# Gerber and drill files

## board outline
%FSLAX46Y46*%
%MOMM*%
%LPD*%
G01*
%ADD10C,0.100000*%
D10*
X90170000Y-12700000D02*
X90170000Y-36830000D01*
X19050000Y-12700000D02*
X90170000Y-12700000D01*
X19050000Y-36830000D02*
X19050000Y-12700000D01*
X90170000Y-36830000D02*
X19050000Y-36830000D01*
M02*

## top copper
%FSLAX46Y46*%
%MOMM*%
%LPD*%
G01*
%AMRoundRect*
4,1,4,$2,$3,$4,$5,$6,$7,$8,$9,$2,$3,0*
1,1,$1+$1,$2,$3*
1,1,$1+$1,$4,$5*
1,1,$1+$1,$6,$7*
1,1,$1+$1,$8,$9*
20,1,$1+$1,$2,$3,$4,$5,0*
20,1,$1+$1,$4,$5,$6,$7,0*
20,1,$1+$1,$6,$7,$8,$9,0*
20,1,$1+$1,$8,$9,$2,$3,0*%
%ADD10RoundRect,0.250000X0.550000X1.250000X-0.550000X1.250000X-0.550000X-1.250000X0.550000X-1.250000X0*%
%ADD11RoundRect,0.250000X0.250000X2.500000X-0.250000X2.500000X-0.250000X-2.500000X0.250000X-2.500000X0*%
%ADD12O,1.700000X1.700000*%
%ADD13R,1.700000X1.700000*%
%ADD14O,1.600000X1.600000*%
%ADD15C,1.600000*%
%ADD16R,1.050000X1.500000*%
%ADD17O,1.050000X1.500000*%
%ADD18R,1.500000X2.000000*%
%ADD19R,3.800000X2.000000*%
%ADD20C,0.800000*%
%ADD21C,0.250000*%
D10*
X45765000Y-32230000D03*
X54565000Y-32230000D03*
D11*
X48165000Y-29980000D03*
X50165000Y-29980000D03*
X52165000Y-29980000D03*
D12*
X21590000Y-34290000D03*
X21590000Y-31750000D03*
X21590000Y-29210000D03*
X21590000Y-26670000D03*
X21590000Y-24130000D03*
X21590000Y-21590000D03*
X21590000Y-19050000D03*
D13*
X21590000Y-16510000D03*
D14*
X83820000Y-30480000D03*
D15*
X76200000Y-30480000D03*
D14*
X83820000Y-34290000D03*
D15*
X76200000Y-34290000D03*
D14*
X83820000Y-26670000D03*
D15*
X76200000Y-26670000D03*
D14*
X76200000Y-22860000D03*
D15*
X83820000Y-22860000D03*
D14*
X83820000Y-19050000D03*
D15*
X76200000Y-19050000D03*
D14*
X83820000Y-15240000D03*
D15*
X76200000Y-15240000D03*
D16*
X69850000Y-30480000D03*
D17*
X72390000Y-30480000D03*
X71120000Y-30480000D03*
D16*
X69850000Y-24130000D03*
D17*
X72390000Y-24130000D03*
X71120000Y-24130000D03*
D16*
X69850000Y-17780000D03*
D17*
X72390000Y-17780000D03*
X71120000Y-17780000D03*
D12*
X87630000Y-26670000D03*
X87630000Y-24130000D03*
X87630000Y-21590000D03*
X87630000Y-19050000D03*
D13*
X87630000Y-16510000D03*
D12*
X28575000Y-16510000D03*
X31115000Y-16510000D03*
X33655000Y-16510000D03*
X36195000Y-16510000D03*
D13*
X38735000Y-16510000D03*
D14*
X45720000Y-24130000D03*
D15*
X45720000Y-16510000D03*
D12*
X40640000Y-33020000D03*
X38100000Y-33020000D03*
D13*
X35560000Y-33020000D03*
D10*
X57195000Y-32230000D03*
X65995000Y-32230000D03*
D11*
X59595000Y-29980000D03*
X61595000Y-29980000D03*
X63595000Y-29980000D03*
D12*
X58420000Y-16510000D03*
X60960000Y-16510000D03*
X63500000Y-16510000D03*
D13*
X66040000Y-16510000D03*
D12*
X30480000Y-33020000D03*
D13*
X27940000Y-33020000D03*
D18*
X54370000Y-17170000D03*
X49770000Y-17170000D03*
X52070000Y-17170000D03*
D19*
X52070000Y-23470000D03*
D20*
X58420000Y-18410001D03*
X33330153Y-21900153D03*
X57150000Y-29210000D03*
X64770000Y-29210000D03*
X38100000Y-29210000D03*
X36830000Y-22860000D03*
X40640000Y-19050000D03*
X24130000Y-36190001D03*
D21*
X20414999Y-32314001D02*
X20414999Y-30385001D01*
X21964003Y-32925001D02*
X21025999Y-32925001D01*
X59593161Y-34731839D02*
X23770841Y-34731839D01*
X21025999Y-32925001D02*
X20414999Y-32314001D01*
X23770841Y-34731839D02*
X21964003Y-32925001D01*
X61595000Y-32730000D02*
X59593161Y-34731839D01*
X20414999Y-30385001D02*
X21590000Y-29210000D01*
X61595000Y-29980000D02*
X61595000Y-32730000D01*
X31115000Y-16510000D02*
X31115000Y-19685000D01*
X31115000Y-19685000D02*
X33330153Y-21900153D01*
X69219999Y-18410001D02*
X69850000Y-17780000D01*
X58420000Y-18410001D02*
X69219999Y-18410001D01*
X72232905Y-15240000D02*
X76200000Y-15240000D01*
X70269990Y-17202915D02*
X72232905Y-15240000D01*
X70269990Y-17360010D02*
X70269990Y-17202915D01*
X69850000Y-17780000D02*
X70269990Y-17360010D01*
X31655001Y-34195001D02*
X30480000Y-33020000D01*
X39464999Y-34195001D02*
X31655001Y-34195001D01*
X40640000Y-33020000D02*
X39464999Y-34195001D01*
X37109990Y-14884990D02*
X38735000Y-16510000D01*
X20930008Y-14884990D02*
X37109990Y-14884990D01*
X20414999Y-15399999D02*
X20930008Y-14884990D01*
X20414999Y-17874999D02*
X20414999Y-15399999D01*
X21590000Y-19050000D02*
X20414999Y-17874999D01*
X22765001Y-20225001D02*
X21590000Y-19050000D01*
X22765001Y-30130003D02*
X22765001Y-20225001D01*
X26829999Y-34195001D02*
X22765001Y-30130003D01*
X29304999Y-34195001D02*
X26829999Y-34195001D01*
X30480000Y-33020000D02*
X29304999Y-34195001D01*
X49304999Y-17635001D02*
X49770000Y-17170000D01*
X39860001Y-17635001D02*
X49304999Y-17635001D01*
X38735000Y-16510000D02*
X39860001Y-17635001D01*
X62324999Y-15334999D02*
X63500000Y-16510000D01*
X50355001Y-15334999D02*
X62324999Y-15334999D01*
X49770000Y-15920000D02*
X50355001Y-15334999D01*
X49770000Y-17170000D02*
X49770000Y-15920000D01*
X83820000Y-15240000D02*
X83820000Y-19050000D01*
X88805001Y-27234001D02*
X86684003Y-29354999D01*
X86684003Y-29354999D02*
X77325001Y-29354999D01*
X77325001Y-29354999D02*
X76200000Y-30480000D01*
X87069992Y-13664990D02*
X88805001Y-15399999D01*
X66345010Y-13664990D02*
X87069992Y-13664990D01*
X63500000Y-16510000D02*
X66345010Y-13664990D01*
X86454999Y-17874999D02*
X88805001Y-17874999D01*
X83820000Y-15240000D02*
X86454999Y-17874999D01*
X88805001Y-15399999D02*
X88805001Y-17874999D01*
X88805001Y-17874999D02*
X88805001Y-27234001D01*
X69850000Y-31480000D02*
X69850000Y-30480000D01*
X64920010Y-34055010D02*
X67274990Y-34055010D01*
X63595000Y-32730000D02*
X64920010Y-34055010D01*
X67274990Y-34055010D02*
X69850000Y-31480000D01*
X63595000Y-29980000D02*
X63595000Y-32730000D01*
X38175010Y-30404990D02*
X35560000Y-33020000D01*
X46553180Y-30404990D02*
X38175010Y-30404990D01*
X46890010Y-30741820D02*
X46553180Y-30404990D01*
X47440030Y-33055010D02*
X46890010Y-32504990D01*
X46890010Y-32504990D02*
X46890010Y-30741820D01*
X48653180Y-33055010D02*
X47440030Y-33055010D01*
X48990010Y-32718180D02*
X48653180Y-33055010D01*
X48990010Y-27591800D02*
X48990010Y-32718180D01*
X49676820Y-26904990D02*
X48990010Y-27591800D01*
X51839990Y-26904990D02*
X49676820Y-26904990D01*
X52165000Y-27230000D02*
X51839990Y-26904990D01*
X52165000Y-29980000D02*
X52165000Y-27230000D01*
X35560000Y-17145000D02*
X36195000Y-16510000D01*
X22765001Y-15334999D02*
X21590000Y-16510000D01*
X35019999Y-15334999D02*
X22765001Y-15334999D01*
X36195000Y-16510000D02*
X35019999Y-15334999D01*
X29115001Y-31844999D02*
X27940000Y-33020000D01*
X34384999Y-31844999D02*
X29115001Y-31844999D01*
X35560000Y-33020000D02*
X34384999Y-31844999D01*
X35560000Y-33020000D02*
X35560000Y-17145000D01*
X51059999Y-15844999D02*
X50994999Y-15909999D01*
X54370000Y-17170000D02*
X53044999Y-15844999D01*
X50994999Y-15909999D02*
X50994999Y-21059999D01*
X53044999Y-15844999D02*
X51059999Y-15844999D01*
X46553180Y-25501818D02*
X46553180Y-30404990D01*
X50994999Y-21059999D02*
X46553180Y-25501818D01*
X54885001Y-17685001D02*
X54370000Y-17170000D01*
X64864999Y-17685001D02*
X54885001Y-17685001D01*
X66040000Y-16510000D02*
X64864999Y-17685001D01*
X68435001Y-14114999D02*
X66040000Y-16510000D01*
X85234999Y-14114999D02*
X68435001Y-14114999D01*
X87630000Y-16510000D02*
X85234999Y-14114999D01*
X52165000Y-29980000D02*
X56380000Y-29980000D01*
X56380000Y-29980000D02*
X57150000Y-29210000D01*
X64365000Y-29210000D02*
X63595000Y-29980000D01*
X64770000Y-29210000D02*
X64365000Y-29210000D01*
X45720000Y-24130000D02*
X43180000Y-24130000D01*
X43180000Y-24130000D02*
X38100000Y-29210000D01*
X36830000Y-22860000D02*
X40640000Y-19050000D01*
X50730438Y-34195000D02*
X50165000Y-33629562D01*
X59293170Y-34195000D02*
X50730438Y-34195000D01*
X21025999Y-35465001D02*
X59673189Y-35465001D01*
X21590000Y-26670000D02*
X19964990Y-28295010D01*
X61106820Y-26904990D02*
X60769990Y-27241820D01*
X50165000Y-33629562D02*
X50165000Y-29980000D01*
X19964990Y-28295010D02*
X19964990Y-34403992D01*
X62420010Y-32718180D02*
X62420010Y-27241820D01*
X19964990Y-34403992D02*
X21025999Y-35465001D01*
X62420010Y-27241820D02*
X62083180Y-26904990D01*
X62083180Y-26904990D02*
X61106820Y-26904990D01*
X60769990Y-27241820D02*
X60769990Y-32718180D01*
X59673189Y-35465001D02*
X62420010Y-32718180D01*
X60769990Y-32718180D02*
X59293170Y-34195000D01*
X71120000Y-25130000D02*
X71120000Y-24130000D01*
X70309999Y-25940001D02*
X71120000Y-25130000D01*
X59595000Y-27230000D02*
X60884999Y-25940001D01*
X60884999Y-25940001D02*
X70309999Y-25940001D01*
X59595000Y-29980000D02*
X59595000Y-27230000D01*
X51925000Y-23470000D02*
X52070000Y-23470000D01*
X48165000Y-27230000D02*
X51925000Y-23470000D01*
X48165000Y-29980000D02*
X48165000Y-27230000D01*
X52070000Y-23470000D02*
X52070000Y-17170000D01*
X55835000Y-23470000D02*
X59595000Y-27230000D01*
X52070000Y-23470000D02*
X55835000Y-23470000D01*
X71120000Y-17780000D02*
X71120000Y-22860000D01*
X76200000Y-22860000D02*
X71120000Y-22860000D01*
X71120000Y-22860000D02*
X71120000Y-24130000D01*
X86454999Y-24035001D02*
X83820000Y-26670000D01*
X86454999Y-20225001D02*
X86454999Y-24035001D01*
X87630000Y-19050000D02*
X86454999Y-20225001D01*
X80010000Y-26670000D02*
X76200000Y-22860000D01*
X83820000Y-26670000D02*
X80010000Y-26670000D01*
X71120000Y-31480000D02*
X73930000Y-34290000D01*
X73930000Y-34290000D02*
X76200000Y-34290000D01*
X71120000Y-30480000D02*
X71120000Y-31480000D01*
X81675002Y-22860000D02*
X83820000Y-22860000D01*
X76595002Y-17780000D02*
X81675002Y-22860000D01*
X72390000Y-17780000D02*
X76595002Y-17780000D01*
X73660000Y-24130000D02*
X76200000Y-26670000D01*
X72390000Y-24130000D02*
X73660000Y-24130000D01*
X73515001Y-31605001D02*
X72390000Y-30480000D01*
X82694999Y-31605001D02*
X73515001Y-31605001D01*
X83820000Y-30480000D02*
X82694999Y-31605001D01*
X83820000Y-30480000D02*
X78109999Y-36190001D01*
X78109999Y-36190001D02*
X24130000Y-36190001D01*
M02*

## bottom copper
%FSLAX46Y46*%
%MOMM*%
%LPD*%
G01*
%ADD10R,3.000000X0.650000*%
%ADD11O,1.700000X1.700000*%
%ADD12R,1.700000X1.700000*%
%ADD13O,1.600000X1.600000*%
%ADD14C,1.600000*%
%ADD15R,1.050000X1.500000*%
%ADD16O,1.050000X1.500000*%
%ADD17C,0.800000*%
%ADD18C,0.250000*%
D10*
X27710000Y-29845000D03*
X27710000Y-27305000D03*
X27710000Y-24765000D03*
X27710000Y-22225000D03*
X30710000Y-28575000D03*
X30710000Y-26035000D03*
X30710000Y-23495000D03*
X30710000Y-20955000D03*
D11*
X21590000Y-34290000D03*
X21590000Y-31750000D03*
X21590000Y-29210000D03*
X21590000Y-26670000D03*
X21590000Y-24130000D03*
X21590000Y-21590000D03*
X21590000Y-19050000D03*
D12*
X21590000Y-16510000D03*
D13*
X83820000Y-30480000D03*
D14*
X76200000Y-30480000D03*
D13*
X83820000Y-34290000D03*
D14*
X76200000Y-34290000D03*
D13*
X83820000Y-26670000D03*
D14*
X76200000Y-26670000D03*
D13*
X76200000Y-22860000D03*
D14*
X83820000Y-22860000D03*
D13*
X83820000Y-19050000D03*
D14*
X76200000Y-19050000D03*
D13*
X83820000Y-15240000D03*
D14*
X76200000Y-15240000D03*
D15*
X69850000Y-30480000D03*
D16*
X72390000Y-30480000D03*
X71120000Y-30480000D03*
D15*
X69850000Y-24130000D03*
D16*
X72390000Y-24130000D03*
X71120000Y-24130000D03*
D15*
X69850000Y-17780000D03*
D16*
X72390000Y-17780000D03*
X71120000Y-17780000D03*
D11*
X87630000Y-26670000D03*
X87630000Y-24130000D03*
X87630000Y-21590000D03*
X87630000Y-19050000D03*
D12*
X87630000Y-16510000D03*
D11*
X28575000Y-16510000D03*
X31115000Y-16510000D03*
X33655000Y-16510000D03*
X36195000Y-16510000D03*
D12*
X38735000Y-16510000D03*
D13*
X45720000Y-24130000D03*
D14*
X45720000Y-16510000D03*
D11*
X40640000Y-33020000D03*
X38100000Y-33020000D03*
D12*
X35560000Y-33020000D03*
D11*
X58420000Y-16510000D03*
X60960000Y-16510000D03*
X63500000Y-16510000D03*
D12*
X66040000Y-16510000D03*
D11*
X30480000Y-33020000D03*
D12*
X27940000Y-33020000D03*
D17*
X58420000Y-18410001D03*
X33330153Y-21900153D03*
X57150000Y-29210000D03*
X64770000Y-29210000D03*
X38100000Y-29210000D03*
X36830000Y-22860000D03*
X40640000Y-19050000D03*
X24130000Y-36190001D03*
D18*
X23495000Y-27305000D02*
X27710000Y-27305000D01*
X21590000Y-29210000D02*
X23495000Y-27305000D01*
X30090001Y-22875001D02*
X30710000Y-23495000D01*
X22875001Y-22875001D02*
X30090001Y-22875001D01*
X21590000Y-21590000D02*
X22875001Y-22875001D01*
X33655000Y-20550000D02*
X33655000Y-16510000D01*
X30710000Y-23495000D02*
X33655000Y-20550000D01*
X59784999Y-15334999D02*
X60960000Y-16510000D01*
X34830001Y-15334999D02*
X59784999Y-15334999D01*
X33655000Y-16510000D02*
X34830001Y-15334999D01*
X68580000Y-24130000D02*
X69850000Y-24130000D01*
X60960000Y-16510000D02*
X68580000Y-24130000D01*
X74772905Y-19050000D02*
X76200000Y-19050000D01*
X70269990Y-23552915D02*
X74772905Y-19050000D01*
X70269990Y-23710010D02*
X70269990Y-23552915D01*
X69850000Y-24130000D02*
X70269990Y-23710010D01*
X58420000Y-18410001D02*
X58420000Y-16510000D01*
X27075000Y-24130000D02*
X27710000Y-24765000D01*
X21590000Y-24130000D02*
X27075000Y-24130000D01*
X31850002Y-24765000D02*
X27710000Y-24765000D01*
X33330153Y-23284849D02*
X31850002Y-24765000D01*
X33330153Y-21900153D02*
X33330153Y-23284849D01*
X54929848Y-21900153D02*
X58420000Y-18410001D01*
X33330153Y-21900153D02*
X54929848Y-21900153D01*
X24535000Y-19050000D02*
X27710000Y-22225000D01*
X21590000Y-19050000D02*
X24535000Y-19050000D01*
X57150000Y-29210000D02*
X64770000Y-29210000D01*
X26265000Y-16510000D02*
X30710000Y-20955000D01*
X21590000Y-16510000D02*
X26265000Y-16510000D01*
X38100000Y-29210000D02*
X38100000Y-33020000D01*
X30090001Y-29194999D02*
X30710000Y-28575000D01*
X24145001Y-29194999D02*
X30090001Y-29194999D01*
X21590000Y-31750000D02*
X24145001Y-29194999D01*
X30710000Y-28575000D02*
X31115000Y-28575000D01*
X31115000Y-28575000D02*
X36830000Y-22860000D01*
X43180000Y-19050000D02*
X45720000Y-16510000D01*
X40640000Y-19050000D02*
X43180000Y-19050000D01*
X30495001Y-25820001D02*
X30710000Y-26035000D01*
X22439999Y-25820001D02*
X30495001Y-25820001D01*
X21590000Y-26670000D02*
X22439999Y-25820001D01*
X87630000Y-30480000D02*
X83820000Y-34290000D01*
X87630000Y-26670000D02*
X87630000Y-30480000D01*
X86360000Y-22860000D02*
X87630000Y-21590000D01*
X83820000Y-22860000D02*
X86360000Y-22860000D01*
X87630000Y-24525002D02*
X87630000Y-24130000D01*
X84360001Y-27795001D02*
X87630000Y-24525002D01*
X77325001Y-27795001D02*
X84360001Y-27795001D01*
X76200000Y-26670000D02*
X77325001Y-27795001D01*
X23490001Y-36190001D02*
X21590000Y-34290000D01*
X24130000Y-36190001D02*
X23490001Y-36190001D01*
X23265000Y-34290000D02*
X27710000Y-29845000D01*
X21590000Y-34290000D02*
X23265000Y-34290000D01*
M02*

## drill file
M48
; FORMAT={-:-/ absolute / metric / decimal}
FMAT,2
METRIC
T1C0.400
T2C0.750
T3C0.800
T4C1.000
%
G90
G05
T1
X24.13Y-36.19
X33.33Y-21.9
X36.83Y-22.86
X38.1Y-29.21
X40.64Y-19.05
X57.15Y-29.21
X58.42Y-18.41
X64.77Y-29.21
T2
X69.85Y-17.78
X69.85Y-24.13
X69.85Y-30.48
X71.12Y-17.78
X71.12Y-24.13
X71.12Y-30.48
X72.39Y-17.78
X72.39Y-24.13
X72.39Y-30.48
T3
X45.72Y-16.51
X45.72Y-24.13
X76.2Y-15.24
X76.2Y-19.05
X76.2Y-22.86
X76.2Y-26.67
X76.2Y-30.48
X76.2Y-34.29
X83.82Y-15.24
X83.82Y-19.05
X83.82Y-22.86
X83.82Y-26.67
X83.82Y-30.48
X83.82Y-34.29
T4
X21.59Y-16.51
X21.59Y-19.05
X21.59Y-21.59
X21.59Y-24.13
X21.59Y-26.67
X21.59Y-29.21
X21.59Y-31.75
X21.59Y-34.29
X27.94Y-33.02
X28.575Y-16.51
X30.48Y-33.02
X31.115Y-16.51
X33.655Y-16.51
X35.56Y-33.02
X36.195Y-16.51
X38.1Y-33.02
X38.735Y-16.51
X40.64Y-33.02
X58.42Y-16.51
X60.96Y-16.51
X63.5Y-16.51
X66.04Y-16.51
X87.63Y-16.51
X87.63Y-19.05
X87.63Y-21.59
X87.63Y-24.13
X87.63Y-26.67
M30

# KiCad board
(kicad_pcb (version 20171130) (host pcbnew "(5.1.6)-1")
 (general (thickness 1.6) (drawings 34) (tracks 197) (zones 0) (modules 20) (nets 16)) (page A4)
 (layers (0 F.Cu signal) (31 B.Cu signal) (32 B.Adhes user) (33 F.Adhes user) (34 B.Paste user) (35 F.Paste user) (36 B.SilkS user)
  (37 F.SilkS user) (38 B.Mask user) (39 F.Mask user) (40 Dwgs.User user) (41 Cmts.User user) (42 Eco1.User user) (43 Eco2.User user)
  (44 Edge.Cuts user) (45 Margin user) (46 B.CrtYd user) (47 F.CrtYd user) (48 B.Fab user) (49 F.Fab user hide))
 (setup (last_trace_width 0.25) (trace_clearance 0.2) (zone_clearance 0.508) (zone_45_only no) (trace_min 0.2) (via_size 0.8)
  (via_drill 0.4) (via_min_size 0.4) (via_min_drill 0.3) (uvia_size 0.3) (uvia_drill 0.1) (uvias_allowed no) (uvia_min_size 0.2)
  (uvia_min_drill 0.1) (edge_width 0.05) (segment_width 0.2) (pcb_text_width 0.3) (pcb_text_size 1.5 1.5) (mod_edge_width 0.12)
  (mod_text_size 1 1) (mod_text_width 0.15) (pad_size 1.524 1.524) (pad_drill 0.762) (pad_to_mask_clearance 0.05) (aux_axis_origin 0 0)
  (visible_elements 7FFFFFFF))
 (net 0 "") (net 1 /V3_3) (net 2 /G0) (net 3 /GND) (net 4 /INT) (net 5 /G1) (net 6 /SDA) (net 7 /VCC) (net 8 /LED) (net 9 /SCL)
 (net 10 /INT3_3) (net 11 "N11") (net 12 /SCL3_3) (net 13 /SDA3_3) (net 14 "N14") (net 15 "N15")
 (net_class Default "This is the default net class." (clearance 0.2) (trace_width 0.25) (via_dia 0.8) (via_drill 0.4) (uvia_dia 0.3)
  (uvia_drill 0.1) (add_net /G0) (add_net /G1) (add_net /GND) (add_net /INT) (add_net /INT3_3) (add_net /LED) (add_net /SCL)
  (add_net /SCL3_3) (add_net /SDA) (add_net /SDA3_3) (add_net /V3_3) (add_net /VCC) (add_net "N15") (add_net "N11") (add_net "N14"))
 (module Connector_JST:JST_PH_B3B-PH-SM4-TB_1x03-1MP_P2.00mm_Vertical (layer F.Cu) (at 50.165 30.48 180)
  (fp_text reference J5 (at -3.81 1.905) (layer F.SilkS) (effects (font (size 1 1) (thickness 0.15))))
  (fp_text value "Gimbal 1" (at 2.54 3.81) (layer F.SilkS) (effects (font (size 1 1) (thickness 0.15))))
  (pad MP smd roundrect (at 4.4 -1.75 180) (size 1.6 3) (layers F.Cu F.Paste F.Mask) (roundrect_rratio 0.15625))
  (pad MP smd roundrect (at -4.4 -1.75 180) (size 1.6 3) (layers F.Cu F.Paste F.Mask) (roundrect_rratio 0.15625))
  (pad 3 smd roundrect (at 2 0.5 180) (size 1 5.5) (layers F.Cu F.Paste F.Mask) (roundrect_rratio 0.25) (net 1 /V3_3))
  (pad 2 smd roundrect (at 0 0.5 180) (size 1 5.5) (layers F.Cu F.Paste F.Mask) (roundrect_rratio 0.25) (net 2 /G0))
  (pad 1 smd roundrect (at -2 0.5 180) (size 1 5.5) (layers F.Cu F.Paste F.Mask) (roundrect_rratio 0.25) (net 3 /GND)))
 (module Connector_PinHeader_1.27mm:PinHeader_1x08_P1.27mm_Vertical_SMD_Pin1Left (layer B.Cu) (at 29.21 25.4 180)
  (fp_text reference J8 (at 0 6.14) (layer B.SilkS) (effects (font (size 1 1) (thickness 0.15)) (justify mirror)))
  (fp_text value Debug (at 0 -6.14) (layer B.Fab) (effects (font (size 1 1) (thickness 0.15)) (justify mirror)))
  (pad 8 smd rect (at 1.5 -4.445 180) (size 3 0.65) (layers B.Cu B.Paste B.Mask) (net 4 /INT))
  (pad 6 smd rect (at 1.5 -1.905 180) (size 3 0.65) (layers B.Cu B.Paste B.Mask) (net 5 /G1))
  (pad 4 smd rect (at 1.5 0.635 180) (size 3 0.65) (layers B.Cu B.Paste B.Mask) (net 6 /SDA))
  (pad 2 smd rect (at 1.5 3.175 180) (size 3 0.65) (layers B.Cu B.Paste B.Mask) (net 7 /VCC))
  (pad 7 smd rect (at -1.5 -3.175 180) (size 3 0.65) (layers B.Cu B.Paste B.Mask) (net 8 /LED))
  (pad 5 smd rect (at -1.5 -0.635 180) (size 3 0.65) (layers B.Cu B.Paste B.Mask) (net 2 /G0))
  (pad 3 smd rect (at -1.5 1.905 180) (size 3 0.65) (layers B.Cu B.Paste B.Mask) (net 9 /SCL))
  (pad 1 smd rect (at -1.5 4.445 180) (size 3 0.65) (layers B.Cu B.Paste B.Mask) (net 3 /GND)))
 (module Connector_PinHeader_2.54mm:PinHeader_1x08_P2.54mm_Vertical (layer F.Cu) (at 21.59 16.51)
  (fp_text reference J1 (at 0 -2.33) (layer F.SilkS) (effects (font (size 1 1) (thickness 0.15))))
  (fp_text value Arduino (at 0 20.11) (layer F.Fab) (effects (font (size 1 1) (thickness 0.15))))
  (pad 8 thru_hole oval (at 0 17.78) (size 1.7 1.7) (drill 1) (layers *.Cu *.Mask) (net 4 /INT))
  (pad 7 thru_hole oval (at 0 15.24) (size 1.7 1.7) (drill 1) (layers *.Cu *.Mask) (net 8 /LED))
  (pad 6 thru_hole oval (at 0 12.7) (size 1.7 1.7) (drill 1) (layers *.Cu *.Mask) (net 5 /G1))
  (pad 5 thru_hole oval (at 0 10.16) (size 1.7 1.7) (drill 1) (layers *.Cu *.Mask) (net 2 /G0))
  (pad 4 thru_hole oval (at 0 7.62) (size 1.7 1.7) (drill 1) (layers *.Cu *.Mask) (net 6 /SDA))
  (pad 3 thru_hole oval (at 0 5.08) (size 1.7 1.7) (drill 1) (layers *.Cu *.Mask) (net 9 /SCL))
  (pad 2 thru_hole oval (at 0 2.54) (size 1.7 1.7) (drill 1) (layers *.Cu *.Mask) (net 7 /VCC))
  (pad 1 thru_hole rect (at 0 0) (size 1.7 1.7) (drill 1) (layers *.Cu *.Mask) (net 3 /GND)))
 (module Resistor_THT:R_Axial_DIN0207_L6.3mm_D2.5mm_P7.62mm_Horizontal (layer F.Cu) (at 76.2 30.48)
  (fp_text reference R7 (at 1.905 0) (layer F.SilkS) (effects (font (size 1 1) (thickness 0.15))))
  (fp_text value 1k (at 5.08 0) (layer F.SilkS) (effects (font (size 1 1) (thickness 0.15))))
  (pad 2 thru_hole oval (at 7.62 0) (size 1.6 1.6) (drill 0.8) (layers *.Cu *.Mask) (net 4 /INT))
  (pad 1 thru_hole circle (at 0 0) (size 1.6 1.6) (drill 0.8) (layers *.Cu *.Mask) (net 7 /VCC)))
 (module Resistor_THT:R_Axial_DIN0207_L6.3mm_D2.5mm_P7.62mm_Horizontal (layer F.Cu) (at 76.2 34.29)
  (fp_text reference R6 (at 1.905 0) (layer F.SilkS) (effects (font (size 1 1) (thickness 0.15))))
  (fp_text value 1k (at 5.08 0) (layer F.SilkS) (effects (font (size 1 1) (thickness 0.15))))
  (pad 2 thru_hole oval (at 7.62 0) (size 1.6 1.6) (drill 0.8) (layers *.Cu *.Mask) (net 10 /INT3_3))
  (pad 1 thru_hole circle (at 0 0) (size 1.6 1.6) (drill 0.8) (layers *.Cu *.Mask) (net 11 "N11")))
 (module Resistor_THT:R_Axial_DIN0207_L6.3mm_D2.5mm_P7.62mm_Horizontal (layer F.Cu) (at 76.2 26.67)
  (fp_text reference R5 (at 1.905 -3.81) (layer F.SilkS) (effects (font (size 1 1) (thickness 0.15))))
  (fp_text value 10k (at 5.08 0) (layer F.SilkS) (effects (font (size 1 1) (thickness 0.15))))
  (pad 2 thru_hole oval (at 7.62 0) (size 1.6 1.6) (drill 0.8) (layers *.Cu *.Mask) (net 1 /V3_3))
  (pad 1 thru_hole circle (at 0 0) (size 1.6 1.6) (drill 0.8) (layers *.Cu *.Mask) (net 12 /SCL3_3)))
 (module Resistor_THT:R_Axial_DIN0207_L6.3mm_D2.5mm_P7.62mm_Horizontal (layer F.Cu) (at 83.82 22.86 180)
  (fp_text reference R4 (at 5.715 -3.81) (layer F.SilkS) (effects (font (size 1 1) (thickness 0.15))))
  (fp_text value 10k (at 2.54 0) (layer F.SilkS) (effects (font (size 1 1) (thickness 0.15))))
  (pad 2 thru_hole oval (at 7.62 0 180) (size 1.6 1.6) (drill 0.8) (layers *.Cu *.Mask) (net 1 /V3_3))
  (pad 1 thru_hole circle (at 0 0 180) (size 1.6 1.6) (drill 0.8) (layers *.Cu *.Mask) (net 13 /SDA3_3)))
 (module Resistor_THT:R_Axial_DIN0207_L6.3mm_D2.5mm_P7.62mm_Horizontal (layer F.Cu) (at 76.2 19.05)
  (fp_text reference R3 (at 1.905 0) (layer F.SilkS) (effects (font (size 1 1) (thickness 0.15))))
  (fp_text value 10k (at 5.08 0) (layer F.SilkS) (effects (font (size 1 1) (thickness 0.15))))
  (pad 2 thru_hole oval (at 7.62 0) (size 1.6 1.6) (drill 0.8) (layers *.Cu *.Mask) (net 7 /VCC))
  (pad 1 thru_hole circle (at 0 0) (size 1.6 1.6) (drill 0.8) (layers *.Cu *.Mask) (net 9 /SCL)))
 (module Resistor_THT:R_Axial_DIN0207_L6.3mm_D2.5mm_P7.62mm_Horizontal (layer F.Cu) (at 76.2 15.24)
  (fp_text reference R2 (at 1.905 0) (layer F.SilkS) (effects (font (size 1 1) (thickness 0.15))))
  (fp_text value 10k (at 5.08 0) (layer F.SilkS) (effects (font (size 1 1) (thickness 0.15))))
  (pad 2 thru_hole oval (at 7.62 0) (size 1.6 1.6) (drill 0.8) (layers *.Cu *.Mask) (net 7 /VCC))
  (pad 1 thru_hole circle (at 0 0) (size 1.6 1.6) (drill 0.8) (layers *.Cu *.Mask) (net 6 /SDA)))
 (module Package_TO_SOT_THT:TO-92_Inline (layer F.Cu) (at 69.85 30.48)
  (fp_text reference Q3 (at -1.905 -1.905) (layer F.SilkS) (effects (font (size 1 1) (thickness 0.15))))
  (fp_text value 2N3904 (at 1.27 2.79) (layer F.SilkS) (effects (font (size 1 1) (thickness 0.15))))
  (pad 1 thru_hole rect (at 0 0) (size 1.05 1.5) (drill 0.75) (layers *.Cu *.Mask) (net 3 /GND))
  (pad 3 thru_hole oval (at 2.54 0) (size 1.05 1.5) (drill 0.75) (layers *.Cu *.Mask) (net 4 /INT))
  (pad 2 thru_hole oval (at 1.27 0) (size 1.05 1.5) (drill 0.75) (layers *.Cu *.Mask) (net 11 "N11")))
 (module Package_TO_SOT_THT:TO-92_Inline (layer F.Cu) (at 69.85 24.13)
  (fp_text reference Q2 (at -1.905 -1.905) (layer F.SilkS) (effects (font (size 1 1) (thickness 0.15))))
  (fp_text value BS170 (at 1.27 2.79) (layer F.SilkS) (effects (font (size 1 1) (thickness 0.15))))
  (pad 1 thru_hole rect (at 0 0) (size 1.05 1.5) (drill 0.75) (layers *.Cu *.Mask) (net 9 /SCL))
  (pad 3 thru_hole oval (at 2.54 0) (size 1.05 1.5) (drill 0.75) (layers *.Cu *.Mask) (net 12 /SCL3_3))
  (pad 2 thru_hole oval (at 1.27 0) (size 1.05 1.5) (drill 0.75) (layers *.Cu *.Mask) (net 1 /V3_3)))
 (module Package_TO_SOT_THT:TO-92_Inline (layer F.Cu) (at 69.85 17.78)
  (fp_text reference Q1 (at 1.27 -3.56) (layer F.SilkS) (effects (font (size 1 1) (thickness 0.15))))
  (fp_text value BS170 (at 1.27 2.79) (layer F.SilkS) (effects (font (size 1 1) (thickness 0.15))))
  (pad 1 thru_hole rect (at 0 0) (size 1.05 1.5) (drill 0.75) (layers *.Cu *.Mask) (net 6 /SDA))
  (pad 3 thru_hole oval (at 2.54 0) (size 1.05 1.5) (drill 0.75) (layers *.Cu *.Mask) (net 13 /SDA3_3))
  (pad 2 thru_hole oval (at 1.27 0) (size 1.05 1.5) (drill 0.75) (layers *.Cu *.Mask) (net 1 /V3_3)))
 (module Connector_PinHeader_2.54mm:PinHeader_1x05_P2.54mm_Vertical (layer F.Cu) (at 87.63 16.51)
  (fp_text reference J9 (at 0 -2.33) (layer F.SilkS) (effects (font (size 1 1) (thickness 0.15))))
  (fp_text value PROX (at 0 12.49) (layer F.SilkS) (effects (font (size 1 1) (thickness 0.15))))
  (pad 5 thru_hole oval (at 0 10.16) (size 1.7 1.7) (drill 1) (layers *.Cu *.Mask) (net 10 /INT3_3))
  (pad 4 thru_hole oval (at 0 7.62) (size 1.7 1.7) (drill 1) (layers *.Cu *.Mask) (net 12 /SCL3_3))
  (pad 3 thru_hole oval (at 0 5.08) (size 1.7 1.7) (drill 1) (layers *.Cu *.Mask) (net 13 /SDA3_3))
  (pad 2 thru_hole oval (at 0 2.54) (size 1.7 1.7) (drill 1) (layers *.Cu *.Mask) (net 1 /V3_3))
  (pad 1 thru_hole rect (at 0 0) (size 1.7 1.7) (drill 1) (layers *.Cu *.Mask) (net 3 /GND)))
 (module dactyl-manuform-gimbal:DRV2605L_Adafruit (layer F.Cu) (at 38.735 16.51 270)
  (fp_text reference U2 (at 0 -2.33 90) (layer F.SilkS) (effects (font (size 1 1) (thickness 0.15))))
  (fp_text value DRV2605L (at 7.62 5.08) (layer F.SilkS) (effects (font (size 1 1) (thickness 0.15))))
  (pad 5 thru_hole oval (at 0 10.16 270) (size 1.7 1.7) (drill 1) (layers *.Cu *.Mask) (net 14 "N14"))
  (pad 4 thru_hole oval (at 0 7.62 270) (size 1.7 1.7) (drill 1) (layers *.Cu *.Mask) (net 6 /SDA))
  (pad 3 thru_hole oval (at 0 5.08 270) (size 1.7 1.7) (drill 1) (layers *.Cu *.Mask) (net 9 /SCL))
  (pad 2 thru_hole oval (at 0 2.54 270) (size 1.7 1.7) (drill 1) (layers *.Cu *.Mask) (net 3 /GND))
  (pad 1 thru_hole rect (at 0 0 270) (size 1.7 1.7) (drill 1) (layers *.Cu *.Mask) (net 7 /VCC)))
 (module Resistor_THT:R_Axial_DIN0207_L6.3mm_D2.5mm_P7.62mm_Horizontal (layer F.Cu) (at 45.72 16.51 270)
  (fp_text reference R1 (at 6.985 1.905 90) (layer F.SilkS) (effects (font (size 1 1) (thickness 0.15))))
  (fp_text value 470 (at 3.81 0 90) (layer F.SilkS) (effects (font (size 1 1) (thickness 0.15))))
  (pad 2 thru_hole oval (at 7.62 0 270) (size 1.6 1.6) (drill 0.8) (layers *.Cu *.Mask) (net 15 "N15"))
  (pad 1 thru_hole circle (at 0 0 270) (size 1.6 1.6) (drill 0.8) (layers *.Cu *.Mask) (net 8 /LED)))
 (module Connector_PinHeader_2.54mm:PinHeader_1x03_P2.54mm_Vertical (layer F.Cu) (at 35.56 33.02 90)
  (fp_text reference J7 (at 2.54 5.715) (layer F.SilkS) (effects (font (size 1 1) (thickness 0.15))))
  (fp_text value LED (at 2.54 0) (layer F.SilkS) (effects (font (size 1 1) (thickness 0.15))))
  (pad 3 thru_hole oval (at 0 5.08 90) (size 1.7 1.7) (drill 1) (layers *.Cu *.Mask) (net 7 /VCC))
  (pad 2 thru_hole oval (at 0 2.54 90) (size 1.7 1.7) (drill 1) (layers *.Cu *.Mask) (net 15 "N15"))
  (pad 1 thru_hole rect (at 0 0 90) (size 1.7 1.7) (drill 1) (layers *.Cu *.Mask) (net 3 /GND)))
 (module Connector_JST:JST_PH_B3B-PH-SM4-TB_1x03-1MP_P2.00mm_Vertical (layer F.Cu) (at 61.595 30.48 180)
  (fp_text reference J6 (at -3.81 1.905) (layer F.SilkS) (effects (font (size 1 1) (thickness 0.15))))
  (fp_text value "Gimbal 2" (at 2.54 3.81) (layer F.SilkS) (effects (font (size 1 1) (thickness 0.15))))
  (pad MP smd roundrect (at 4.4 -1.75 180) (size 1.6 3) (layers F.Cu F.Paste F.Mask) (roundrect_rratio 0.15625))
  (pad MP smd roundrect (at -4.4 -1.75 180) (size 1.6 3) (layers F.Cu F.Paste F.Mask) (roundrect_rratio 0.15625))
  (pad 3 smd roundrect (at 2 0.5 180) (size 1 5.5) (layers F.Cu F.Paste F.Mask) (roundrect_rratio 0.25) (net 1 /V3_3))
  (pad 2 smd roundrect (at 0 0.5 180) (size 1 5.5) (layers F.Cu F.Paste F.Mask) (roundrect_rratio 0.25) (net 5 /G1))
  (pad 1 smd roundrect (at -2 0.5 180) (size 1 5.5) (layers F.Cu F.Paste F.Mask) (roundrect_rratio 0.25) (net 3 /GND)))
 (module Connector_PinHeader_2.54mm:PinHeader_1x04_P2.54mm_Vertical (layer F.Cu) (at 66.04 16.51 270)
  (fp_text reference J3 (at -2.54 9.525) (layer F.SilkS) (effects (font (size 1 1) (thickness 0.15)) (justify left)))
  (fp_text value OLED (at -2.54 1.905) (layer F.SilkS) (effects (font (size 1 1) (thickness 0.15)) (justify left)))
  (pad 4 thru_hole oval (at 0 7.62 270) (size 1.7 1.7) (drill 1) (layers *.Cu *.Mask) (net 6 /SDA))
  (pad 3 thru_hole oval (at 0 5.08 270) (size 1.7 1.7) (drill 1) (layers *.Cu *.Mask) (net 9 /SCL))
  (pad 2 thru_hole oval (at 0 2.54 270) (size 1.7 1.7) (drill 1) (layers *.Cu *.Mask) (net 7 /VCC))
  (pad 1 thru_hole rect (at 0 0 270) (size 1.7 1.7) (drill 1) (layers *.Cu *.Mask) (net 3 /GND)))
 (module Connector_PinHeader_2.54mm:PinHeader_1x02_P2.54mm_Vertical (layer F.Cu) (at 27.94 33.02 90)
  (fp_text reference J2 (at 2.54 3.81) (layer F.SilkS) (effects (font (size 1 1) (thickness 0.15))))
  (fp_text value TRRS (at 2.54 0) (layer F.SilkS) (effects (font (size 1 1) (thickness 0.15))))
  (pad 2 thru_hole oval (at 0 2.54 90) (size 1.7 1.7) (drill 1) (layers *.Cu *.Mask) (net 7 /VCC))
  (pad 1 thru_hole rect (at 0 0 90) (size 1.7 1.7) (drill 1) (layers *.Cu *.Mask) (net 3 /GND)))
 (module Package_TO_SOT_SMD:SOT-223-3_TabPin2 (layer F.Cu) (at 52.07 20.32 270)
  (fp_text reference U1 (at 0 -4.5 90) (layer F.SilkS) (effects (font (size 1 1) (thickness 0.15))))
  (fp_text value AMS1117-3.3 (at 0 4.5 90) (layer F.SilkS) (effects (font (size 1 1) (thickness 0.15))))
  (pad 1 smd rect (at -3.15 -2.3 270) (size 2 1.5) (layers F.Cu F.Paste F.Mask) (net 3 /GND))
  (pad 3 smd rect (at -3.15 2.3 270) (size 2 1.5) (layers F.Cu F.Paste F.Mask) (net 7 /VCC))
  (pad 2 smd rect (at -3.15 0 270) (size 2 1.5) (layers F.Cu F.Paste F.Mask) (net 1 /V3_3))
  (pad 2 smd rect (at 3.15 0 270) (size 2 3.8) (layers F.Cu F.Paste F.Mask) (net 1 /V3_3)))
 (gr_line (start 90.17 12.7) (end 90.17 36.83) (layer Edge.Cuts) (width 0.1))
 (gr_line (start 19.05 12.7) (end 90.17 12.7) (layer Edge.Cuts) (width 0.1))
 (gr_line (start 19.05 36.83) (end 19.05 12.7) (layer Edge.Cuts) (width 0.1))
 (gr_line (start 90.17 36.83) (end 19.05 36.83) (layer Edge.Cuts) (width 0.1))
 (segment (start 20.414999 32.314001) (end 20.414999 30.385001) (width 0.25) (layer F.Cu) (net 5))
 (segment (start 21.964003 32.925001) (end 21.025999 32.925001) (width 0.25) (layer F.Cu) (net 5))
 (segment (start 59.593161 34.731839) (end 23.770841 34.731839) (width 0.25) (layer F.Cu) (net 5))
 (segment (start 21.025999 32.925001) (end 20.414999 32.314001) (width 0.25) (layer F.Cu) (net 5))
 (segment (start 23.770841 34.731839) (end 21.964003 32.925001) (width 0.25) (layer F.Cu) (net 5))
 (segment (start 61.595 32.73) (end 59.593161 34.731839) (width 0.25) (layer F.Cu) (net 5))
 (segment (start 20.414999 30.385001) (end 21.59 29.21) (width 0.25) (layer F.Cu) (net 5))
 (segment (start 61.595 29.98) (end 61.595 32.73) (width 0.25) (layer F.Cu) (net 5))
 (segment (start 23.495 27.305) (end 27.71 27.305) (width 0.25) (layer B.Cu) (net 5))
 (segment (start 21.59 29.21) (end 23.495 27.305) (width 0.25) (layer B.Cu) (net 5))
 (segment (start 30.090001 22.875001) (end 30.71 23.495) (width 0.25) (layer B.Cu) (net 9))
 (segment (start 22.875001 22.875001) (end 30.090001 22.875001) (width 0.25) (layer B.Cu) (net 9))
 (segment (start 21.59 21.59) (end 22.875001 22.875001) (width 0.25) (layer B.Cu) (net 9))
 (segment (start 33.655 20.55) (end 33.655 16.51) (width 0.25) (layer B.Cu) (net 9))
 (segment (start 30.71 23.495) (end 33.655 20.55) (width 0.25) (layer B.Cu) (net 9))
 (segment (start 59.784999 15.334999) (end 60.96 16.51) (width 0.25) (layer B.Cu) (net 9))
 (segment (start 34.830001 15.334999) (end 59.784999 15.334999) (width 0.25) (layer B.Cu) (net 9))
 (segment (start 33.655 16.51) (end 34.830001 15.334999) (width 0.25) (layer B.Cu) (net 9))
 (segment (start 68.58 24.13) (end 69.85 24.13) (width 0.25) (layer B.Cu) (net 9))
 (segment (start 60.96 16.51) (end 68.58 24.13) (width 0.25) (layer B.Cu) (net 9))
 (segment (start 74.772905 19.05) (end 76.2 19.05) (width 0.25) (layer B.Cu) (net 9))
 (segment (start 70.26999 23.552915) (end 74.772905 19.05) (width 0.25) (layer B.Cu) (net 9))
 (segment (start 70.26999 23.71001) (end 70.26999 23.552915) (width 0.25) (layer B.Cu) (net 9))
 (segment (start 69.85 24.13) (end 70.26999 23.71001) (width 0.25) (layer B.Cu) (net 9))
 (via (at 58.42 18.410001) (size 0.8) (drill 0.4) (layers F.Cu B.Cu) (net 6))
 (segment (start 58.42 18.410001) (end 58.42 16.51) (width 0.25) (layer B.Cu) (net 6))
 (segment (start 27.075 24.13) (end 27.71 24.765) (width 0.25) (layer B.Cu) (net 6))
 (segment (start 21.59 24.13) (end 27.075 24.13) (width 0.25) (layer B.Cu) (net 6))
 (via (at 33.330153 21.900153) (size 0.8) (drill 0.4) (layers F.Cu B.Cu) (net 6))
 (segment (start 31.115 16.51) (end 31.115 19.685) (width 0.25) (layer F.Cu) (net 6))
 (segment (start 31.115 19.685) (end 33.330153 21.900153) (width 0.25) (layer F.Cu) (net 6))
 (segment (start 31.850002 24.765) (end 27.71 24.765) (width 0.25) (layer B.Cu) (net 6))
 (segment (start 33.330153 23.284849) (end 31.850002 24.765) (width 0.25) (layer B.Cu) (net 6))
 (segment (start 33.330153 21.900153) (end 33.330153 23.284849) (width 0.25) (layer B.Cu) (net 6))
 (segment (start 54.929848 21.900153) (end 58.42 18.410001) (width 0.25) (layer B.Cu) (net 6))
 (segment (start 33.330153 21.900153) (end 54.929848 21.900153) (width 0.25) (layer B.Cu) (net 6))
 (segment (start 69.219999 18.410001) (end 69.85 17.78) (width 0.25) (layer F.Cu) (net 6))
 (segment (start 58.42 18.410001) (end 69.219999 18.410001) (width 0.25) (layer F.Cu) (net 6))
 (segment (start 72.232905 15.24) (end 76.2 15.24) (width 0.25) (layer F.Cu) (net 6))
 (segment (start 70.26999 17.202915) (end 72.232905 15.24) (width 0.25) (layer F.Cu) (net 6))
 (segment (start 70.26999 17.36001) (end 70.26999 17.202915) (width 0.25) (layer F.Cu) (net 6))
 (segment (start 69.85 17.78) (end 70.26999 17.36001) (width 0.25) (layer F.Cu) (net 6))
 (segment (start 31.655001 34.195001) (end 30.48 33.02) (width 0.25) (layer F.Cu) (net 7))
 (segment (start 39.464999 34.195001) (end 31.655001 34.195001) (width 0.25) (layer F.Cu) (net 7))
 (segment (start 40.64 33.02) (end 39.464999 34.195001) (width 0.25) (layer F.Cu) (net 7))
 (segment (start 37.10999 14.88499) (end 38.735 16.51) (width 0.25) (layer F.Cu) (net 7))
 (segment (start 20.930008 14.88499) (end 37.10999 14.88499) (width 0.25) (layer F.Cu) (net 7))
 (segment (start 20.414999 15.399999) (end 20.930008 14.88499) (width 0.25) (layer F.Cu) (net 7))
 (segment (start 20.414999 17.874999) (end 20.414999 15.399999) (width 0.25) (layer F.Cu) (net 7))
 (segment (start 21.59 19.05) (end 20.414999 17.874999) (width 0.25) (layer F.Cu) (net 7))
 (segment (start 22.765001 20.225001) (end 21.59 19.05) (width 0.25) (layer F.Cu) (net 7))
 (segment (start 22.765001 30.130003) (end 22.765001 20.225001) (width 0.25) (layer F.Cu) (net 7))
 (segment (start 26.829999 34.195001) (end 22.765001 30.130003) (width 0.25) (layer F.Cu) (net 7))
 (segment (start 29.304999 34.195001) (end 26.829999 34.195001) (width 0.25) (layer F.Cu) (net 7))
 (segment (start 30.48 33.02) (end 29.304999 34.195001) (width 0.25) (layer F.Cu) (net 7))
 (segment (start 49.304999 17.635001) (end 49.77 17.17) (width 0.25) (layer F.Cu) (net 7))
 (segment (start 39.860001 17.635001) (end 49.304999 17.635001) (width 0.25) (layer F.Cu) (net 7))
 (segment (start 38.735 16.51) (end 39.860001 17.635001) (width 0.25) (layer F.Cu) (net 7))
 (segment (start 62.324999 15.334999) (end 63.5 16.51) (width 0.25) (layer F.Cu) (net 7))
 (segment (start 50.355001 15.334999) (end 62.324999 15.334999) (width 0.25) (layer F.Cu) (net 7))
 (segment (start 49.77 15.92) (end 50.355001 15.334999) (width 0.25) (layer F.Cu) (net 7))
 (segment (start 49.77 17.17) (end 49.77 15.92) (width 0.25) (layer F.Cu) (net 7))
 (segment (start 83.82 15.24) (end 83.82 19.05) (width 0.25) (layer F.Cu) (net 7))
 (segment (start 88.805001 27.234001) (end 86.684003 29.354999) (width 0.25) (layer F.Cu) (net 7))
 (segment (start 86.684003 29.354999) (end 77.325001 29.354999) (width 0.25) (layer F.Cu) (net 7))
 (segment (start 77.325001 29.354999) (end 76.2 30.48) (width 0.25) (layer F.Cu) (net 7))
 (segment (start 87.069992 13.66499) (end 88.805001 15.399999) (width 0.25) (layer F.Cu) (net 7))
 (segment (start 66.34501 13.66499) (end 87.069992 13.66499) (width 0.25) (layer F.Cu) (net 7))
 (segment (start 63.5 16.51) (end 66.34501 13.66499) (width 0.25) (layer F.Cu) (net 7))
 (segment (start 86.454999 17.874999) (end 88.805001 17.874999) (width 0.25) (layer F.Cu) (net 7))
 (segment (start 83.82 15.24) (end 86.454999 17.874999) (width 0.25) (layer F.Cu) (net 7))
 (segment (start 88.805001 15.399999) (end 88.805001 17.874999) (width 0.25) (layer F.Cu) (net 7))
 (segment (start 88.805001 17.874999) (end 88.805001 27.234001) (width 0.25) (layer F.Cu) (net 7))
 (segment (start 24.535 19.05) (end 27.71 22.225) (width 0.25) (layer B.Cu) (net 7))
 (segment (start 21.59 19.05) (end 24.535 19.05) (width 0.25) (layer B.Cu) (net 7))
 (segment (start 69.85 31.48) (end 69.85 30.48) (width 0.25) (layer F.Cu) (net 3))
 (segment (start 64.92001 34.05501) (end 67.27499 34.05501) (width 0.25) (layer F.Cu) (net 3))
 (segment (start 63.595 32.73) (end 64.92001 34.05501) (width 0.25) (layer F.Cu) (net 3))
 (segment (start 67.27499 34.05501) (end 69.85 31.48) (width 0.25) (layer F.Cu) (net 3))
 (segment (start 63.595 29.98) (end 63.595 32.73) (width 0.25) (layer F.Cu) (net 3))
 (segment (start 38.17501 30.40499) (end 35.56 33.02) (width 0.25) (layer F.Cu) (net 3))
 (segment (start 46.55318 30.40499) (end 38.17501 30.40499) (width 0.25) (layer F.Cu) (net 3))
 (segment (start 46.89001 30.74182) (end 46.55318 30.40499) (width 0.25) (layer F.Cu) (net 3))
 (segment (start 47.44003 33.05501) (end 46.89001 32.50499) (width 0.25) (layer F.Cu) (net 3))
 (segment (start 46.89001 32.50499) (end 46.89001 30.74182) (width 0.25) (layer F.Cu) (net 3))
 (segment (start 48.65318 33.05501) (end 47.44003 33.05501) (width 0.25) (layer F.Cu) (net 3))
 (segment (start 48.99001 32.71818) (end 48.65318 33.05501) (width 0.25) (layer F.Cu) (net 3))
 (segment (start 48.99001 27.5918) (end 48.99001 32.71818) (width 0.25) (layer F.Cu) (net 3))
 (segment (start 49.67682 26.90499) (end 48.99001 27.5918) (width 0.25) (layer F.Cu) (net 3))
 (segment (start 51.83999 26.90499) (end 49.67682 26.90499) (width 0.25) (layer F.Cu) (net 3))
 (segment (start 52.165 27.23) (end 51.83999 26.90499) (width 0.25) (layer F.Cu) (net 3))
 (segment (start 52.165 29.98) (end 52.165 27.23) (width 0.25) (layer F.Cu) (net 3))
 (segment (start 35.56 17.145) (end 36.195 16.51) (width 0.25) (layer F.Cu) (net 3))
 (segment (start 22.765001 15.334999) (end 21.59 16.51) (width 0.25) (layer F.Cu) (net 3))
 (segment (start 35.019999 15.334999) (end 22.765001 15.334999) (width 0.25) (layer F.Cu) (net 3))
 (segment (start 36.195 16.51) (end 35.019999 15.334999) (width 0.25) (layer F.Cu) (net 3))
 (segment (start 29.115001 31.844999) (end 27.94 33.02) (width 0.25) (layer F.Cu) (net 3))
 (segment (start 34.384999 31.844999) (end 29.115001 31.844999) (width 0.25) (layer F.Cu) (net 3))
 (segment (start 35.56 33.02) (end 34.384999 31.844999) (width 0.25) (layer F.Cu) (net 3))
 (segment (start 35.56 33.02) (end 35.56 17.145) (width 0.25) (layer F.Cu) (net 3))
 (segment (start 51.059999 15.844999) (end 50.994999 15.909999) (width 0.25) (layer F.Cu) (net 3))
 (segment (start 54.37 17.17) (end 53.044999 15.844999) (width 0.25) (layer F.Cu) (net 3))
 (segment (start 50.994999 15.909999) (end 50.994999 21.059999) (width 0.25) (layer F.Cu) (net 3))
 (segment (start 53.044999 15.844999) (end 51.059999 15.844999) (width 0.25) (layer F.Cu) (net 3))
 (segment (start 46.55318 25.501818) (end 46.55318 30.40499) (width 0.25) (layer F.Cu) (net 3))
 (segment (start 50.994999 21.059999) (end 46.55318 25.501818) (width 0.25) (layer F.Cu) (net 3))
 (segment (start 54.885001 17.685001) (end 54.37 17.17) (width 0.25) (layer F.Cu) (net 3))
 (segment (start 64.864999 17.685001) (end 54.885001 17.685001) (width 0.25) (layer F.Cu) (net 3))
 (segment (start 66.04 16.51) (end 64.864999 17.685001) (width 0.25) (layer F.Cu) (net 3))
 (segment (start 68.435001 14.114999) (end 66.04 16.51) (width 0.25) (layer F.Cu) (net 3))
 (segment (start 85.234999 14.114999) (end 68.435001 14.114999) (width 0.25) (layer F.Cu) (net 3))
 (segment (start 87.63 16.51) (end 85.234999 14.114999) (width 0.25) (layer F.Cu) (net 3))
 (via (at 57.15 29.21) (size 0.8) (drill 0.4) (layers F.Cu B.Cu) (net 3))
 (segment (start 52.165 29.98) (end 56.38 29.98) (width 0.25) (layer F.Cu) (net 3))
 (segment (start 56.38 29.98) (end 57.15 29.21) (width 0.25) (layer F.Cu) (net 3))
 (via (at 64.77 29.21) (size 0.8) (drill 0.4) (layers F.Cu B.Cu) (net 3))
 (segment (start 57.15 29.21) (end 64.77 29.21) (width 0.25) (layer B.Cu) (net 3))
 (segment (start 64.365 29.21) (end 63.595 29.98) (width 0.25) (layer F.Cu) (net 3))
 (segment (start 64.77 29.21) (end 64.365 29.21) (width 0.25) (layer F.Cu) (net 3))
 (segment (start 26.265 16.51) (end 30.71 20.955) (width 0.25) (layer B.Cu) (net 3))
 (segment (start 21.59 16.51) (end 26.265 16.51) (width 0.25) (layer B.Cu) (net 3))
 (via (at 38.1 29.21) (size 0.8) (drill 0.4) (layers F.Cu B.Cu) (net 15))
 (segment (start 45.72 24.13) (end 43.18 24.13) (width 0.25) (layer F.Cu) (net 15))
 (segment (start 43.18 24.13) (end 38.1 29.21) (width 0.25) (layer F.Cu) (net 15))
 (segment (start 38.1 29.21) (end 38.1 33.02) (width 0.25) (layer B.Cu) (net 15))
 (segment (start 30.090001 29.194999) (end 30.71 28.575) (width 0.25) (layer B.Cu) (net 8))
 (segment (start 24.145001 29.194999) (end 30.090001 29.194999) (width 0.25) (layer B.Cu) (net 8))
 (segment (start 21.59 31.75) (end 24.145001 29.194999) (width 0.25) (layer B.Cu) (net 8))
 (via (at 36.83 22.86) (size 0.8) (drill 0.4) (layers F.Cu B.Cu) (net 8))
 (segment (start 30.71 28.575) (end 31.115 28.575) (width 0.25) (layer B.Cu) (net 8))
 (segment (start 31.115 28.575) (end 36.83 22.86) (width 0.25) (layer B.Cu) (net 8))
 (via (at 40.64 19.05) (size 0.8) (drill 0.4) (layers F.Cu B.Cu) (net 8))
 (segment (start 36.83 22.86) (end 40.64 19.05) (width 0.25) (layer F.Cu) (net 8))
 (segment (start 43.18 19.05) (end 45.72 16.51) (width 0.25) (layer B.Cu) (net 8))
 (segment (start 40.64 19.05) (end 43.18 19.05) (width 0.25) (layer B.Cu) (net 8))
 (segment (start 50.730438 34.195) (end 50.165 33.629562) (width 0.25) (layer F.Cu) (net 2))
 (segment (start 59.29317 34.195) (end 50.730438 34.195) (width 0.25) (layer F.Cu) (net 2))
 (segment (start 21.025999 35.465001) (end 59.673189 35.465001) (width 0.25) (layer F.Cu) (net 2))
 (segment (start 21.59 26.67) (end 19.96499 28.29501) (width 0.25) (layer F.Cu) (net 2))
 (segment (start 61.10682 26.90499) (end 60.76999 27.24182) (width 0.25) (layer F.Cu) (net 2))
 (segment (start 50.165 33.629562) (end 50.165 29.98) (width 0.25) (layer F.Cu) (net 2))
 (segment (start 19.96499 28.29501) (end 19.96499 34.403992) (width 0.25) (layer F.Cu) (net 2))
 (segment (start 62.42001 32.71818) (end 62.42001 27.24182) (width 0.25) (layer F.Cu) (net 2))
 (segment (start 19.96499 34.403992) (end 21.025999 35.465001) (width 0.25) (layer F.Cu) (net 2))
 (segment (start 62.42001 27.24182) (end 62.08318 26.90499) (width 0.25) (layer F.Cu) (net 2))
 (segment (start 62.08318 26.90499) (end 61.10682 26.90499) (width 0.25) (layer F.Cu) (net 2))
 (segment (start 60.76999 27.24182) (end 60.76999 32.71818) (width 0.25) (layer F.Cu) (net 2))
 (segment (start 59.673189 35.465001) (end 62.42001 32.71818) (width 0.25) (layer F.Cu) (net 2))
 (segment (start 60.76999 32.71818) (end 59.29317 34.195) (width 0.25) (layer F.Cu) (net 2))
 (segment (start 30.495001 25.820001) (end 30.71 26.035) (width 0.25) (layer B.Cu) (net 2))
 (segment (start 22.439999 25.820001) (end 30.495001 25.820001) (width 0.25) (layer B.Cu) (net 2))
 (segment (start 21.59 26.67) (end 22.439999 25.820001) (width 0.25) (layer B.Cu) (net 2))
 (segment (start 71.12 25.13) (end 71.12 24.13) (width 0.25) (layer F.Cu) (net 1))
 (segment (start 70.309999 25.940001) (end 71.12 25.13) (width 0.25) (layer F.Cu) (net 1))
 (segment (start 59.595 27.23) (end 60.884999 25.940001) (width 0.25) (layer F.Cu) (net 1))
 (segment (start 60.884999 25.940001) (end 70.309999 25.940001) (width 0.25) (layer F.Cu) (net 1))
 (segment (start 59.595 29.98) (end 59.595 27.23) (width 0.25) (layer F.Cu) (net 1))
 (segment (start 51.925 23.47) (end 52.07 23.47) (width 0.25) (layer F.Cu) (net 1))
 (segment (start 48.165 27.23) (end 51.925 23.47) (width 0.25) (layer F.Cu) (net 1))
 (segment (start 48.165 29.98) (end 48.165 27.23) (width 0.25) (layer F.Cu) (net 1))
 (segment (start 52.07 23.47) (end 52.07 17.17) (width 0.25) (layer F.Cu) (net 1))
 (segment (start 55.835 23.47) (end 59.595 27.23) (width 0.25) (layer F.Cu) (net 1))
 (segment (start 52.07 23.47) (end 55.835 23.47) (width 0.25) (layer F.Cu) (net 1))
 (segment (start 71.12 17.78) (end 71.12 22.86) (width 0.25) (layer F.Cu) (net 1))
 (segment (start 76.2 22.86) (end 71.12 22.86) (width 0.25) (layer F.Cu) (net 1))
 (segment (start 71.12 22.86) (end 71.12 24.13) (width 0.25) (layer F.Cu) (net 1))
 (segment (start 86.454999 24.035001) (end 83.82 26.67) (width 0.25) (layer F.Cu) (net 1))
 (segment (start 86.454999 20.225001) (end 86.454999 24.035001) (width 0.25) (layer F.Cu) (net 1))
 (segment (start 87.63 19.05) (end 86.454999 20.225001) (width 0.25) (layer F.Cu) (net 1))
 (segment (start 80.01 26.67) (end 76.2 22.86) (width 0.25) (layer F.Cu) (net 1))
 (segment (start 83.82 26.67) (end 80.01 26.67) (width 0.25) (layer F.Cu) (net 1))
 (segment (start 71.12 31.48) (end 73.93 34.29) (width 0.25) (layer F.Cu) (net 11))
 (segment (start 73.93 34.29) (end 76.2 34.29) (width 0.25) (layer F.Cu) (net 11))
 (segment (start 71.12 30.48) (end 71.12 31.48) (width 0.25) (layer F.Cu) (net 11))
 (segment (start 87.63 30.48) (end 83.82 34.29) (width 0.25) (layer B.Cu) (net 10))
 (segment (start 87.63 26.67) (end 87.63 30.48) (width 0.25) (layer B.Cu) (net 10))
 (segment (start 81.675002 22.86) (end 83.82 22.86) (width 0.25) (layer F.Cu) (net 13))
 (segment (start 76.595002 17.78) (end 81.675002 22.86) (width 0.25) (layer F.Cu) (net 13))
 (segment (start 72.39 17.78) (end 76.595002 17.78) (width 0.25) (layer F.Cu) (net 13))
 (segment (start 86.36 22.86) (end 87.63 21.59) (width 0.25) (layer B.Cu) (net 13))
 (segment (start 83.82 22.86) (end 86.36 22.86) (width 0.25) (layer B.Cu) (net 13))
 (segment (start 73.66 24.13) (end 76.2 26.67) (width 0.25) (layer F.Cu) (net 12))
 (segment (start 72.39 24.13) (end 73.66 24.13) (width 0.25) (layer F.Cu) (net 12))
 (segment (start 87.63 24.525002) (end 87.63 24.13) (width 0.25) (layer B.Cu) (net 12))
 (segment (start 84.360001 27.795001) (end 87.63 24.525002) (width 0.25) (layer B.Cu) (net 12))
 (segment (start 77.325001 27.795001) (end 84.360001 27.795001) (width 0.25) (layer B.Cu) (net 12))
 (segment (start 76.2 26.67) (end 77.325001 27.795001) (width 0.25) (layer B.Cu) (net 12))
 (segment (start 73.515001 31.605001) (end 72.39 30.48) (width 0.25) (layer F.Cu) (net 4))
 (segment (start 82.694999 31.605001) (end 73.515001 31.605001) (width 0.25) (layer F.Cu) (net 4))
 (segment (start 83.82 30.48) (end 82.694999 31.605001) (width 0.25) (layer F.Cu) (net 4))
 (via (at 24.13 36.190001) (size 0.8) (drill 0.4) (layers F.Cu B.Cu) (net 4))
 (segment (start 83.82 30.48) (end 78.109999 36.190001) (width 0.25) (layer F.Cu) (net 4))
 (segment (start 78.109999 36.190001) (end 24.13 36.190001) (width 0.25) (layer F.Cu) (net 4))
 (segment (start 23.490001 36.190001) (end 21.59 34.29) (width 0.25) (layer B.Cu) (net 4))
 (segment (start 24.13 36.190001) (end 23.490001 36.190001) (width 0.25) (layer B.Cu) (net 4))
 (segment (start 23.265 34.29) (end 27.71 29.845) (width 0.25) (layer B.Cu) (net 4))
 (segment (start 21.59 34.29) (end 23.265 34.29) (width 0.25) (layer B.Cu) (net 4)))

